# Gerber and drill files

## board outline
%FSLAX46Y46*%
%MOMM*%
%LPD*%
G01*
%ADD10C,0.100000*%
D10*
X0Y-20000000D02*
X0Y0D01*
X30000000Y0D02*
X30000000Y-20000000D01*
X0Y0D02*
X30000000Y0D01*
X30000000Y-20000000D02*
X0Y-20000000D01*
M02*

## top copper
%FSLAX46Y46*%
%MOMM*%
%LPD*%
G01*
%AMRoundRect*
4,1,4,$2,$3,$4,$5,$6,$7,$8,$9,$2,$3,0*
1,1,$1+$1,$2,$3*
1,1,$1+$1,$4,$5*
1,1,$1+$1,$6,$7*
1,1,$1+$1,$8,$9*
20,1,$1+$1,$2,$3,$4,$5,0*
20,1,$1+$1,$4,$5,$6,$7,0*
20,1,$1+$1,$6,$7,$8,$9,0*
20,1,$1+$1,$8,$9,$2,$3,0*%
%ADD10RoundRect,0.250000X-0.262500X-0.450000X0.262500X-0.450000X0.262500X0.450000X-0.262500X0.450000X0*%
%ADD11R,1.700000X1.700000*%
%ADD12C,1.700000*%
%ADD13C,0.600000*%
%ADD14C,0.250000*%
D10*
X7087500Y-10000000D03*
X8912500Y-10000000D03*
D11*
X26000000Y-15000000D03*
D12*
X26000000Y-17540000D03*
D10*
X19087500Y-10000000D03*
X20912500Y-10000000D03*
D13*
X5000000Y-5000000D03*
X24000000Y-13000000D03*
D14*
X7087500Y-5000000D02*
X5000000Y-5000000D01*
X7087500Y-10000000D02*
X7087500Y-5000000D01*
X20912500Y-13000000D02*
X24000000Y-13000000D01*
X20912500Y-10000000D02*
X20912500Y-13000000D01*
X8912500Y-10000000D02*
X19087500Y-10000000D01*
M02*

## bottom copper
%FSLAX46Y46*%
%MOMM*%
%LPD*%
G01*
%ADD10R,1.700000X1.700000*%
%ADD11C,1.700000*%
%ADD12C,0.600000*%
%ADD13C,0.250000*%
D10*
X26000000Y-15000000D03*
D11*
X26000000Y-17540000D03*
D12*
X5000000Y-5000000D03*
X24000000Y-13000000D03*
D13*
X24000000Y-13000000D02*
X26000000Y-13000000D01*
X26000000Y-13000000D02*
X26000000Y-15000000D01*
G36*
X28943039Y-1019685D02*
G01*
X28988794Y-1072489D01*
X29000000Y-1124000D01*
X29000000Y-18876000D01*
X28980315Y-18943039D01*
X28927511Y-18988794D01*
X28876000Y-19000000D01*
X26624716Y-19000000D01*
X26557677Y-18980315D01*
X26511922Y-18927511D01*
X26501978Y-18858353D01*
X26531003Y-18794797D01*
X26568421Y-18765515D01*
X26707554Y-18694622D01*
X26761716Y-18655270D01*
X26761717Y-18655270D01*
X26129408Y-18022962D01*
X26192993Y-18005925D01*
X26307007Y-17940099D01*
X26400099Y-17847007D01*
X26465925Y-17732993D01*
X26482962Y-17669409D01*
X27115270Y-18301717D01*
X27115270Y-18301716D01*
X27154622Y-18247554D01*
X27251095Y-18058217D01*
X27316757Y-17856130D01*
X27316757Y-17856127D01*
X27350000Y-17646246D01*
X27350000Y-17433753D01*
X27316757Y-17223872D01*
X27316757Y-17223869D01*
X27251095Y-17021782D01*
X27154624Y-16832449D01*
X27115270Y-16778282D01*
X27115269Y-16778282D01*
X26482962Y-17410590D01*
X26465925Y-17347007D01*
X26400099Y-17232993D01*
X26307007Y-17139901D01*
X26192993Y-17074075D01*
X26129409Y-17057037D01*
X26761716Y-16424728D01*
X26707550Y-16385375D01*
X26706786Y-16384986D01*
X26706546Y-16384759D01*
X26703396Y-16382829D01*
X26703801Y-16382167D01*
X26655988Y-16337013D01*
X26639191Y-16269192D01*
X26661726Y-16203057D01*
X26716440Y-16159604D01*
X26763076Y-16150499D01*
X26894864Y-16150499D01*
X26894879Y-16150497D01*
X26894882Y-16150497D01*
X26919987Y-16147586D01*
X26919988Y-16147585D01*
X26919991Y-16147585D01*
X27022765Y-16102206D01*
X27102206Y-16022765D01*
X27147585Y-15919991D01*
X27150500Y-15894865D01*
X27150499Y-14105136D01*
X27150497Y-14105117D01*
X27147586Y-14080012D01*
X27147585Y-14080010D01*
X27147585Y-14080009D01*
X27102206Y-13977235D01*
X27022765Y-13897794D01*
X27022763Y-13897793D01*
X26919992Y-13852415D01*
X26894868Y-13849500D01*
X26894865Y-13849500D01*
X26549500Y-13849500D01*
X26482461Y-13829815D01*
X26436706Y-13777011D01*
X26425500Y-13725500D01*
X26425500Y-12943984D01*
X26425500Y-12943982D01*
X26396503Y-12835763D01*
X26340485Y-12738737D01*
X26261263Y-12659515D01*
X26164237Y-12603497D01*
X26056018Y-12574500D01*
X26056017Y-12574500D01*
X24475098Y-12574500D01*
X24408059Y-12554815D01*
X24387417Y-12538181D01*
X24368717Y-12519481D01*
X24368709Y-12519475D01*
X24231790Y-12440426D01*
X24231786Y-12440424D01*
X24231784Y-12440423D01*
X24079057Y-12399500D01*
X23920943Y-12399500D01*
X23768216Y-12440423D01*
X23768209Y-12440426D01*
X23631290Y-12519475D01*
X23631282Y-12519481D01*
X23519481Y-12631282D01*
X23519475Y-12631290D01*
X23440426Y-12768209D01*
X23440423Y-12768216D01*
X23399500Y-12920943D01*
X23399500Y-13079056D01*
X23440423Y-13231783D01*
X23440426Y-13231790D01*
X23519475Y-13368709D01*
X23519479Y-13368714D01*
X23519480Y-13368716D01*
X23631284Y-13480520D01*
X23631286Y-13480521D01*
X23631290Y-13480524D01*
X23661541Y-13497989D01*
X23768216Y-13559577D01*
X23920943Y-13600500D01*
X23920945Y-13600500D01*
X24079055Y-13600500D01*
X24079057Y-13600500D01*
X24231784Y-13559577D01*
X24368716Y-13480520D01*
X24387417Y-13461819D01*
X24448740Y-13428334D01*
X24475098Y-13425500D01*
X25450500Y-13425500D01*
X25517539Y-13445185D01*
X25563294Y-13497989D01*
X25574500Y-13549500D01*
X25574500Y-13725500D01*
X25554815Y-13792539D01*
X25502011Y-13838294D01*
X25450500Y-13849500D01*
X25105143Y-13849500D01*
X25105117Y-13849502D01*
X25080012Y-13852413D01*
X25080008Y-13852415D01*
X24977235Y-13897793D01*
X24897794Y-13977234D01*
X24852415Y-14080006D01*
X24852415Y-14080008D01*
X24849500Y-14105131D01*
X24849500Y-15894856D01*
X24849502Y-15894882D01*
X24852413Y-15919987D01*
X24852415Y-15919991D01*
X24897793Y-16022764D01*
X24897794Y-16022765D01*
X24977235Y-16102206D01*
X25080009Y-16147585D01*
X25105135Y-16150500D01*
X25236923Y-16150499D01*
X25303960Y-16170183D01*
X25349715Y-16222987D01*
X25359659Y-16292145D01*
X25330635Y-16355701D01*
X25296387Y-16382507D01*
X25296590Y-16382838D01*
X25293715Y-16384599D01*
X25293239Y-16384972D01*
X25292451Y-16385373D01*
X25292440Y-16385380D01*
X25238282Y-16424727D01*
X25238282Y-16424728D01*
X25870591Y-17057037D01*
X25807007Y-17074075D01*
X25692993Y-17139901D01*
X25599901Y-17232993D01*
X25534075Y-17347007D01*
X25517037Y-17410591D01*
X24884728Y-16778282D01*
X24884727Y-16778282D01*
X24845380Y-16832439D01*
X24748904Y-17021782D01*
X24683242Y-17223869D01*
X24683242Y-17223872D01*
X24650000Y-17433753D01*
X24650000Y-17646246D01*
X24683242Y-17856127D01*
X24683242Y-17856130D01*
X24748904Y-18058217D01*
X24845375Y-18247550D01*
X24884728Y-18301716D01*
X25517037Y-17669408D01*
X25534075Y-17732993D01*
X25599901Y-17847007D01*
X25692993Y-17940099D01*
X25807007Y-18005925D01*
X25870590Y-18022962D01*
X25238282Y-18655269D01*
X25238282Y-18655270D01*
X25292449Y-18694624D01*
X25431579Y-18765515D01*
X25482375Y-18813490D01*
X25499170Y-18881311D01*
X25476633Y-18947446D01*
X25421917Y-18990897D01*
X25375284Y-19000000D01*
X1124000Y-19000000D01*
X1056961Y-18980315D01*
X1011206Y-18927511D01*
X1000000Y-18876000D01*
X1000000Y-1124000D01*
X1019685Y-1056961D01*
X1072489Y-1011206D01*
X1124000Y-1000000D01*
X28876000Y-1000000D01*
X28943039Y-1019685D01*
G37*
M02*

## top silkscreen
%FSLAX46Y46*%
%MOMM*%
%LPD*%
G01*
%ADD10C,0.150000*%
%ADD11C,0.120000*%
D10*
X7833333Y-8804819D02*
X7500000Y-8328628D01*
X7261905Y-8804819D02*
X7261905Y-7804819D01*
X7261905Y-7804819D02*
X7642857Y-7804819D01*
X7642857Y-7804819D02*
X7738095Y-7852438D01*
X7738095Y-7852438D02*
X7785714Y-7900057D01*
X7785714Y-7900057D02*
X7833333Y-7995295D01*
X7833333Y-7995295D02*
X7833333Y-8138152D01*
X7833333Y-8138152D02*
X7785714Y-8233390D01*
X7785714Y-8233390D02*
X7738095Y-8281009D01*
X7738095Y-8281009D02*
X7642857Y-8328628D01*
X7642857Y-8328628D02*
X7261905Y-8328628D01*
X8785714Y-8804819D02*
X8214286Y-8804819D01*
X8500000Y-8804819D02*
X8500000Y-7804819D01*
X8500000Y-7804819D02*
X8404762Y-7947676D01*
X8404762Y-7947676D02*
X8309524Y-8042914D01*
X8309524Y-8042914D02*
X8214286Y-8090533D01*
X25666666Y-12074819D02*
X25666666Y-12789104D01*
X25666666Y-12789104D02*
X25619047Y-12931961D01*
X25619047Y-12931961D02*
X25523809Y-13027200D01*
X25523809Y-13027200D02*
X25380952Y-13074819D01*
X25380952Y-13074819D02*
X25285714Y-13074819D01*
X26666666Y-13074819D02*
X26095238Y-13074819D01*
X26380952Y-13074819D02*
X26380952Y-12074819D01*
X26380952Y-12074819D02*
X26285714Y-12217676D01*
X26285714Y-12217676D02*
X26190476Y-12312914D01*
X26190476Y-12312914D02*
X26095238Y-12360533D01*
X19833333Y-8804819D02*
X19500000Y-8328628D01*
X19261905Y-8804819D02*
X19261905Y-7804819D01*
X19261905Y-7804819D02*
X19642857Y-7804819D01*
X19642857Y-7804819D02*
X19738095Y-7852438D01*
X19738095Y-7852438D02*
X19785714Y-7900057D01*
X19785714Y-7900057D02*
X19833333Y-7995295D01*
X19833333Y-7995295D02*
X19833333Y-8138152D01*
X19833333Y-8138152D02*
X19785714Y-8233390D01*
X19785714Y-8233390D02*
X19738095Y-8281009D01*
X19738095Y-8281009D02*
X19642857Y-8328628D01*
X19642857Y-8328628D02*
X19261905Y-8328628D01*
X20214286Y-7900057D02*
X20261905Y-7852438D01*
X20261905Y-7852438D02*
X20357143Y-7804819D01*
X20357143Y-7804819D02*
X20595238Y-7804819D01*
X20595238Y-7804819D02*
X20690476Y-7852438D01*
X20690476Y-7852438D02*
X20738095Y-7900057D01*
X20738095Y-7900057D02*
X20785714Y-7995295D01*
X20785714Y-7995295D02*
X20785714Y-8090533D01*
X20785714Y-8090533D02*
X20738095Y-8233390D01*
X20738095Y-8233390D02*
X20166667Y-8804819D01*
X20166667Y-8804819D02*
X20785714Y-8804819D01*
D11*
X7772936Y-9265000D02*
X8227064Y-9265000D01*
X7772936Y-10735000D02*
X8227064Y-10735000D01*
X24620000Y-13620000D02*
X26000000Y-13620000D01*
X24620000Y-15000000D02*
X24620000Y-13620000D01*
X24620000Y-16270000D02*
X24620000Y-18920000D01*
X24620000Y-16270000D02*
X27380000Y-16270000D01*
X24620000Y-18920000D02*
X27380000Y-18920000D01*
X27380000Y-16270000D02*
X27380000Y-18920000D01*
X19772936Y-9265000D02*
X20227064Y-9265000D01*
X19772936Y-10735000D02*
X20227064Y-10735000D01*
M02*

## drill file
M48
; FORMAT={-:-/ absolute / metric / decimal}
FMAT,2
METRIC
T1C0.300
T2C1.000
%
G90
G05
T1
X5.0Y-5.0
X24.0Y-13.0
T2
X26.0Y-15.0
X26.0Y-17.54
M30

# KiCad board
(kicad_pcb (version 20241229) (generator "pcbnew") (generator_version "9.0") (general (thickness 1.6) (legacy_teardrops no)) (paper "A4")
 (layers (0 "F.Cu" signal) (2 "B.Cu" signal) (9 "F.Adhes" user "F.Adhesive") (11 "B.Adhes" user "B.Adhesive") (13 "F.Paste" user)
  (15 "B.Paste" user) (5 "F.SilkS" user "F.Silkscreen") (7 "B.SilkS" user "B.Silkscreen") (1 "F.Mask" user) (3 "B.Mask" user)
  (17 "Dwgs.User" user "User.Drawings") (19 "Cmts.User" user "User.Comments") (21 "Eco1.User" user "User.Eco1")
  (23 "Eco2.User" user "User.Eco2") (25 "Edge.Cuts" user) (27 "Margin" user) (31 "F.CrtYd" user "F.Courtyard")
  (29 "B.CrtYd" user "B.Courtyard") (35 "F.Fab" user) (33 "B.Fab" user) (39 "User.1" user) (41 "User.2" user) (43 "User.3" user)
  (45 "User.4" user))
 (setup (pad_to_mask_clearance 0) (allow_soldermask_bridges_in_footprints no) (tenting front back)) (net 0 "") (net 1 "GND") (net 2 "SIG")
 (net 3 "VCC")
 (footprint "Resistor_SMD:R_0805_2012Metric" (layer "F.Cu") (at 8 10)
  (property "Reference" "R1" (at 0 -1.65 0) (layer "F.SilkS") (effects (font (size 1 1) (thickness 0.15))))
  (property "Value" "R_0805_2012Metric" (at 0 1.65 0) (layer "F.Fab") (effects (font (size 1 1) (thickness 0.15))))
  (fp_line (start -0.227064 -0.735) (end 0.227064 -0.735) (stroke (width 0.12) (type solid)) (layer "F.SilkS"))
  (fp_line (start -0.227064 0.735) (end 0.227064 0.735) (stroke (width 0.12) (type solid)) (layer "F.SilkS"))
  (pad "1" smd roundrect (at -0.9125 0) (size 1.025 1.4) (layers "F.Cu" "F.Mask" "F.Paste") (roundrect_rratio 0.243902) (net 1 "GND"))
  (pad "2" smd roundrect (at 0.9125 0) (size 1.025 1.4) (layers "F.Cu" "F.Mask" "F.Paste") (roundrect_rratio 0.243902) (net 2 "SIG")))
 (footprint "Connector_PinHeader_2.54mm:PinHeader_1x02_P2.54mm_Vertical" (layer "F.Cu") (at 26 15)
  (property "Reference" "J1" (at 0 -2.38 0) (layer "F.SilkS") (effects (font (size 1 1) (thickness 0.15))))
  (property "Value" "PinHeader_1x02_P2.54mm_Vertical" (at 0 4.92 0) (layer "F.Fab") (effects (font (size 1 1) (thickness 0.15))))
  (fp_line (start -1.38 -1.38) (end 0 -1.38) (stroke (width 0.12) (type solid)) (layer "F.SilkS"))
  (fp_line (start -1.38 0) (end -1.38 -1.38) (stroke (width 0.12) (type solid)) (layer "F.SilkS"))
  (fp_line (start -1.38 1.27) (end -1.38 3.92) (stroke (width 0.12) (type solid)) (layer "F.SilkS"))
  (fp_line (start -1.38 1.27) (end 1.38 1.27) (stroke (width 0.12) (type solid)) (layer "F.SilkS"))
  (fp_line (start -1.38 3.92) (end 1.38 3.92) (stroke (width 0.12) (type solid)) (layer "F.SilkS"))
  (fp_line (start 1.38 1.27) (end 1.38 3.92) (stroke (width 0.12) (type solid)) (layer "F.SilkS"))
  (pad "1" thru_hole rect (at 0 0) (size 1.7 1.7) (drill 1) (layers "*.Cu" "*.Mask") (remove_unused_layers no) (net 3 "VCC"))
  (pad "2" thru_hole circle (at 0 2.54) (size 1.7 1.7) (drill 1) (layers "*.Cu" "*.Mask") (remove_unused_layers no) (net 1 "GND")))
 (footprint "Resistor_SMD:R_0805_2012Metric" (layer "F.Cu") (at 20 10)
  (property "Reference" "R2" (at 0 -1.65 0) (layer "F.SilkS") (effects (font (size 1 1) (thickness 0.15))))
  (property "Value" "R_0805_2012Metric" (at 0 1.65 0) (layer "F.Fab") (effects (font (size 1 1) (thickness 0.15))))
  (fp_line (start -0.227064 -0.735) (end 0.227064 -0.735) (stroke (width 0.12) (type solid)) (layer "F.SilkS"))
  (fp_line (start -0.227064 0.735) (end 0.227064 0.735) (stroke (width 0.12) (type solid)) (layer "F.SilkS"))
  (pad "1" smd roundrect (at -0.9125 0) (size 1.025 1.4) (layers "F.Cu" "F.Mask" "F.Paste") (roundrect_rratio 0.243902) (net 2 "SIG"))
  (pad "2" smd roundrect (at 0.9125 0) (size 1.025 1.4) (layers "F.Cu" "F.Mask" "F.Paste") (roundrect_rratio 0.243902) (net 3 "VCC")))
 (gr_line (start 0 20) (end 0 0) (stroke (width 0.1) (type default)) (layer "Edge.Cuts"))
 (gr_line (start 30 0) (end 30 20) (stroke (width 0.1) (type default)) (layer "Edge.Cuts"))
 (gr_line (start 0 0) (end 30 0) (stroke (width 0.1) (type default)) (layer "Edge.Cuts"))
 (gr_line (start 30 20) (end 0 20) (stroke (width 0.1) (type default)) (layer "Edge.Cuts"))
 (segment (start 7.0875 5) (end 5 5) (width 0.25) (layer "F.Cu") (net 1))
 (segment (start 7.0875 10) (end 7.0875 5) (width 0.25) (layer "F.Cu") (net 1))
 (via (at 5 5) (size 0.6) (drill 0.3) (layers "F.Cu" "B.Cu") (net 1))
 (segment (start 20.9125 13) (end 24 13) (width 0.25) (layer "F.Cu") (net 3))
 (segment (start 20.9125 10) (end 20.9125 13) (width 0.25) (layer "F.Cu") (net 3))
 (via (at 24 13) (size 0.6) (drill 0.3) (layers "F.Cu" "B.Cu") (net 3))
 (segment (start 24 13) (end 26 13) (width 0.25) (layer "B.Cu") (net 3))
 (segment (start 26 13) (end 26 15) (width 0.25) (layer "B.Cu") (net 3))
 (segment (start 8.9125 10) (end 19.0875 10) (width 0.25) (layer "F.Cu") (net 2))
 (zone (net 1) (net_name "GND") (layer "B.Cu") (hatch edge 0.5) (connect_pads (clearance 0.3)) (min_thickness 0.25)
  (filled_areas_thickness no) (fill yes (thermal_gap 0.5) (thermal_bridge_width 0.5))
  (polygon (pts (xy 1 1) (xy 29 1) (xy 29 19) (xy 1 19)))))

